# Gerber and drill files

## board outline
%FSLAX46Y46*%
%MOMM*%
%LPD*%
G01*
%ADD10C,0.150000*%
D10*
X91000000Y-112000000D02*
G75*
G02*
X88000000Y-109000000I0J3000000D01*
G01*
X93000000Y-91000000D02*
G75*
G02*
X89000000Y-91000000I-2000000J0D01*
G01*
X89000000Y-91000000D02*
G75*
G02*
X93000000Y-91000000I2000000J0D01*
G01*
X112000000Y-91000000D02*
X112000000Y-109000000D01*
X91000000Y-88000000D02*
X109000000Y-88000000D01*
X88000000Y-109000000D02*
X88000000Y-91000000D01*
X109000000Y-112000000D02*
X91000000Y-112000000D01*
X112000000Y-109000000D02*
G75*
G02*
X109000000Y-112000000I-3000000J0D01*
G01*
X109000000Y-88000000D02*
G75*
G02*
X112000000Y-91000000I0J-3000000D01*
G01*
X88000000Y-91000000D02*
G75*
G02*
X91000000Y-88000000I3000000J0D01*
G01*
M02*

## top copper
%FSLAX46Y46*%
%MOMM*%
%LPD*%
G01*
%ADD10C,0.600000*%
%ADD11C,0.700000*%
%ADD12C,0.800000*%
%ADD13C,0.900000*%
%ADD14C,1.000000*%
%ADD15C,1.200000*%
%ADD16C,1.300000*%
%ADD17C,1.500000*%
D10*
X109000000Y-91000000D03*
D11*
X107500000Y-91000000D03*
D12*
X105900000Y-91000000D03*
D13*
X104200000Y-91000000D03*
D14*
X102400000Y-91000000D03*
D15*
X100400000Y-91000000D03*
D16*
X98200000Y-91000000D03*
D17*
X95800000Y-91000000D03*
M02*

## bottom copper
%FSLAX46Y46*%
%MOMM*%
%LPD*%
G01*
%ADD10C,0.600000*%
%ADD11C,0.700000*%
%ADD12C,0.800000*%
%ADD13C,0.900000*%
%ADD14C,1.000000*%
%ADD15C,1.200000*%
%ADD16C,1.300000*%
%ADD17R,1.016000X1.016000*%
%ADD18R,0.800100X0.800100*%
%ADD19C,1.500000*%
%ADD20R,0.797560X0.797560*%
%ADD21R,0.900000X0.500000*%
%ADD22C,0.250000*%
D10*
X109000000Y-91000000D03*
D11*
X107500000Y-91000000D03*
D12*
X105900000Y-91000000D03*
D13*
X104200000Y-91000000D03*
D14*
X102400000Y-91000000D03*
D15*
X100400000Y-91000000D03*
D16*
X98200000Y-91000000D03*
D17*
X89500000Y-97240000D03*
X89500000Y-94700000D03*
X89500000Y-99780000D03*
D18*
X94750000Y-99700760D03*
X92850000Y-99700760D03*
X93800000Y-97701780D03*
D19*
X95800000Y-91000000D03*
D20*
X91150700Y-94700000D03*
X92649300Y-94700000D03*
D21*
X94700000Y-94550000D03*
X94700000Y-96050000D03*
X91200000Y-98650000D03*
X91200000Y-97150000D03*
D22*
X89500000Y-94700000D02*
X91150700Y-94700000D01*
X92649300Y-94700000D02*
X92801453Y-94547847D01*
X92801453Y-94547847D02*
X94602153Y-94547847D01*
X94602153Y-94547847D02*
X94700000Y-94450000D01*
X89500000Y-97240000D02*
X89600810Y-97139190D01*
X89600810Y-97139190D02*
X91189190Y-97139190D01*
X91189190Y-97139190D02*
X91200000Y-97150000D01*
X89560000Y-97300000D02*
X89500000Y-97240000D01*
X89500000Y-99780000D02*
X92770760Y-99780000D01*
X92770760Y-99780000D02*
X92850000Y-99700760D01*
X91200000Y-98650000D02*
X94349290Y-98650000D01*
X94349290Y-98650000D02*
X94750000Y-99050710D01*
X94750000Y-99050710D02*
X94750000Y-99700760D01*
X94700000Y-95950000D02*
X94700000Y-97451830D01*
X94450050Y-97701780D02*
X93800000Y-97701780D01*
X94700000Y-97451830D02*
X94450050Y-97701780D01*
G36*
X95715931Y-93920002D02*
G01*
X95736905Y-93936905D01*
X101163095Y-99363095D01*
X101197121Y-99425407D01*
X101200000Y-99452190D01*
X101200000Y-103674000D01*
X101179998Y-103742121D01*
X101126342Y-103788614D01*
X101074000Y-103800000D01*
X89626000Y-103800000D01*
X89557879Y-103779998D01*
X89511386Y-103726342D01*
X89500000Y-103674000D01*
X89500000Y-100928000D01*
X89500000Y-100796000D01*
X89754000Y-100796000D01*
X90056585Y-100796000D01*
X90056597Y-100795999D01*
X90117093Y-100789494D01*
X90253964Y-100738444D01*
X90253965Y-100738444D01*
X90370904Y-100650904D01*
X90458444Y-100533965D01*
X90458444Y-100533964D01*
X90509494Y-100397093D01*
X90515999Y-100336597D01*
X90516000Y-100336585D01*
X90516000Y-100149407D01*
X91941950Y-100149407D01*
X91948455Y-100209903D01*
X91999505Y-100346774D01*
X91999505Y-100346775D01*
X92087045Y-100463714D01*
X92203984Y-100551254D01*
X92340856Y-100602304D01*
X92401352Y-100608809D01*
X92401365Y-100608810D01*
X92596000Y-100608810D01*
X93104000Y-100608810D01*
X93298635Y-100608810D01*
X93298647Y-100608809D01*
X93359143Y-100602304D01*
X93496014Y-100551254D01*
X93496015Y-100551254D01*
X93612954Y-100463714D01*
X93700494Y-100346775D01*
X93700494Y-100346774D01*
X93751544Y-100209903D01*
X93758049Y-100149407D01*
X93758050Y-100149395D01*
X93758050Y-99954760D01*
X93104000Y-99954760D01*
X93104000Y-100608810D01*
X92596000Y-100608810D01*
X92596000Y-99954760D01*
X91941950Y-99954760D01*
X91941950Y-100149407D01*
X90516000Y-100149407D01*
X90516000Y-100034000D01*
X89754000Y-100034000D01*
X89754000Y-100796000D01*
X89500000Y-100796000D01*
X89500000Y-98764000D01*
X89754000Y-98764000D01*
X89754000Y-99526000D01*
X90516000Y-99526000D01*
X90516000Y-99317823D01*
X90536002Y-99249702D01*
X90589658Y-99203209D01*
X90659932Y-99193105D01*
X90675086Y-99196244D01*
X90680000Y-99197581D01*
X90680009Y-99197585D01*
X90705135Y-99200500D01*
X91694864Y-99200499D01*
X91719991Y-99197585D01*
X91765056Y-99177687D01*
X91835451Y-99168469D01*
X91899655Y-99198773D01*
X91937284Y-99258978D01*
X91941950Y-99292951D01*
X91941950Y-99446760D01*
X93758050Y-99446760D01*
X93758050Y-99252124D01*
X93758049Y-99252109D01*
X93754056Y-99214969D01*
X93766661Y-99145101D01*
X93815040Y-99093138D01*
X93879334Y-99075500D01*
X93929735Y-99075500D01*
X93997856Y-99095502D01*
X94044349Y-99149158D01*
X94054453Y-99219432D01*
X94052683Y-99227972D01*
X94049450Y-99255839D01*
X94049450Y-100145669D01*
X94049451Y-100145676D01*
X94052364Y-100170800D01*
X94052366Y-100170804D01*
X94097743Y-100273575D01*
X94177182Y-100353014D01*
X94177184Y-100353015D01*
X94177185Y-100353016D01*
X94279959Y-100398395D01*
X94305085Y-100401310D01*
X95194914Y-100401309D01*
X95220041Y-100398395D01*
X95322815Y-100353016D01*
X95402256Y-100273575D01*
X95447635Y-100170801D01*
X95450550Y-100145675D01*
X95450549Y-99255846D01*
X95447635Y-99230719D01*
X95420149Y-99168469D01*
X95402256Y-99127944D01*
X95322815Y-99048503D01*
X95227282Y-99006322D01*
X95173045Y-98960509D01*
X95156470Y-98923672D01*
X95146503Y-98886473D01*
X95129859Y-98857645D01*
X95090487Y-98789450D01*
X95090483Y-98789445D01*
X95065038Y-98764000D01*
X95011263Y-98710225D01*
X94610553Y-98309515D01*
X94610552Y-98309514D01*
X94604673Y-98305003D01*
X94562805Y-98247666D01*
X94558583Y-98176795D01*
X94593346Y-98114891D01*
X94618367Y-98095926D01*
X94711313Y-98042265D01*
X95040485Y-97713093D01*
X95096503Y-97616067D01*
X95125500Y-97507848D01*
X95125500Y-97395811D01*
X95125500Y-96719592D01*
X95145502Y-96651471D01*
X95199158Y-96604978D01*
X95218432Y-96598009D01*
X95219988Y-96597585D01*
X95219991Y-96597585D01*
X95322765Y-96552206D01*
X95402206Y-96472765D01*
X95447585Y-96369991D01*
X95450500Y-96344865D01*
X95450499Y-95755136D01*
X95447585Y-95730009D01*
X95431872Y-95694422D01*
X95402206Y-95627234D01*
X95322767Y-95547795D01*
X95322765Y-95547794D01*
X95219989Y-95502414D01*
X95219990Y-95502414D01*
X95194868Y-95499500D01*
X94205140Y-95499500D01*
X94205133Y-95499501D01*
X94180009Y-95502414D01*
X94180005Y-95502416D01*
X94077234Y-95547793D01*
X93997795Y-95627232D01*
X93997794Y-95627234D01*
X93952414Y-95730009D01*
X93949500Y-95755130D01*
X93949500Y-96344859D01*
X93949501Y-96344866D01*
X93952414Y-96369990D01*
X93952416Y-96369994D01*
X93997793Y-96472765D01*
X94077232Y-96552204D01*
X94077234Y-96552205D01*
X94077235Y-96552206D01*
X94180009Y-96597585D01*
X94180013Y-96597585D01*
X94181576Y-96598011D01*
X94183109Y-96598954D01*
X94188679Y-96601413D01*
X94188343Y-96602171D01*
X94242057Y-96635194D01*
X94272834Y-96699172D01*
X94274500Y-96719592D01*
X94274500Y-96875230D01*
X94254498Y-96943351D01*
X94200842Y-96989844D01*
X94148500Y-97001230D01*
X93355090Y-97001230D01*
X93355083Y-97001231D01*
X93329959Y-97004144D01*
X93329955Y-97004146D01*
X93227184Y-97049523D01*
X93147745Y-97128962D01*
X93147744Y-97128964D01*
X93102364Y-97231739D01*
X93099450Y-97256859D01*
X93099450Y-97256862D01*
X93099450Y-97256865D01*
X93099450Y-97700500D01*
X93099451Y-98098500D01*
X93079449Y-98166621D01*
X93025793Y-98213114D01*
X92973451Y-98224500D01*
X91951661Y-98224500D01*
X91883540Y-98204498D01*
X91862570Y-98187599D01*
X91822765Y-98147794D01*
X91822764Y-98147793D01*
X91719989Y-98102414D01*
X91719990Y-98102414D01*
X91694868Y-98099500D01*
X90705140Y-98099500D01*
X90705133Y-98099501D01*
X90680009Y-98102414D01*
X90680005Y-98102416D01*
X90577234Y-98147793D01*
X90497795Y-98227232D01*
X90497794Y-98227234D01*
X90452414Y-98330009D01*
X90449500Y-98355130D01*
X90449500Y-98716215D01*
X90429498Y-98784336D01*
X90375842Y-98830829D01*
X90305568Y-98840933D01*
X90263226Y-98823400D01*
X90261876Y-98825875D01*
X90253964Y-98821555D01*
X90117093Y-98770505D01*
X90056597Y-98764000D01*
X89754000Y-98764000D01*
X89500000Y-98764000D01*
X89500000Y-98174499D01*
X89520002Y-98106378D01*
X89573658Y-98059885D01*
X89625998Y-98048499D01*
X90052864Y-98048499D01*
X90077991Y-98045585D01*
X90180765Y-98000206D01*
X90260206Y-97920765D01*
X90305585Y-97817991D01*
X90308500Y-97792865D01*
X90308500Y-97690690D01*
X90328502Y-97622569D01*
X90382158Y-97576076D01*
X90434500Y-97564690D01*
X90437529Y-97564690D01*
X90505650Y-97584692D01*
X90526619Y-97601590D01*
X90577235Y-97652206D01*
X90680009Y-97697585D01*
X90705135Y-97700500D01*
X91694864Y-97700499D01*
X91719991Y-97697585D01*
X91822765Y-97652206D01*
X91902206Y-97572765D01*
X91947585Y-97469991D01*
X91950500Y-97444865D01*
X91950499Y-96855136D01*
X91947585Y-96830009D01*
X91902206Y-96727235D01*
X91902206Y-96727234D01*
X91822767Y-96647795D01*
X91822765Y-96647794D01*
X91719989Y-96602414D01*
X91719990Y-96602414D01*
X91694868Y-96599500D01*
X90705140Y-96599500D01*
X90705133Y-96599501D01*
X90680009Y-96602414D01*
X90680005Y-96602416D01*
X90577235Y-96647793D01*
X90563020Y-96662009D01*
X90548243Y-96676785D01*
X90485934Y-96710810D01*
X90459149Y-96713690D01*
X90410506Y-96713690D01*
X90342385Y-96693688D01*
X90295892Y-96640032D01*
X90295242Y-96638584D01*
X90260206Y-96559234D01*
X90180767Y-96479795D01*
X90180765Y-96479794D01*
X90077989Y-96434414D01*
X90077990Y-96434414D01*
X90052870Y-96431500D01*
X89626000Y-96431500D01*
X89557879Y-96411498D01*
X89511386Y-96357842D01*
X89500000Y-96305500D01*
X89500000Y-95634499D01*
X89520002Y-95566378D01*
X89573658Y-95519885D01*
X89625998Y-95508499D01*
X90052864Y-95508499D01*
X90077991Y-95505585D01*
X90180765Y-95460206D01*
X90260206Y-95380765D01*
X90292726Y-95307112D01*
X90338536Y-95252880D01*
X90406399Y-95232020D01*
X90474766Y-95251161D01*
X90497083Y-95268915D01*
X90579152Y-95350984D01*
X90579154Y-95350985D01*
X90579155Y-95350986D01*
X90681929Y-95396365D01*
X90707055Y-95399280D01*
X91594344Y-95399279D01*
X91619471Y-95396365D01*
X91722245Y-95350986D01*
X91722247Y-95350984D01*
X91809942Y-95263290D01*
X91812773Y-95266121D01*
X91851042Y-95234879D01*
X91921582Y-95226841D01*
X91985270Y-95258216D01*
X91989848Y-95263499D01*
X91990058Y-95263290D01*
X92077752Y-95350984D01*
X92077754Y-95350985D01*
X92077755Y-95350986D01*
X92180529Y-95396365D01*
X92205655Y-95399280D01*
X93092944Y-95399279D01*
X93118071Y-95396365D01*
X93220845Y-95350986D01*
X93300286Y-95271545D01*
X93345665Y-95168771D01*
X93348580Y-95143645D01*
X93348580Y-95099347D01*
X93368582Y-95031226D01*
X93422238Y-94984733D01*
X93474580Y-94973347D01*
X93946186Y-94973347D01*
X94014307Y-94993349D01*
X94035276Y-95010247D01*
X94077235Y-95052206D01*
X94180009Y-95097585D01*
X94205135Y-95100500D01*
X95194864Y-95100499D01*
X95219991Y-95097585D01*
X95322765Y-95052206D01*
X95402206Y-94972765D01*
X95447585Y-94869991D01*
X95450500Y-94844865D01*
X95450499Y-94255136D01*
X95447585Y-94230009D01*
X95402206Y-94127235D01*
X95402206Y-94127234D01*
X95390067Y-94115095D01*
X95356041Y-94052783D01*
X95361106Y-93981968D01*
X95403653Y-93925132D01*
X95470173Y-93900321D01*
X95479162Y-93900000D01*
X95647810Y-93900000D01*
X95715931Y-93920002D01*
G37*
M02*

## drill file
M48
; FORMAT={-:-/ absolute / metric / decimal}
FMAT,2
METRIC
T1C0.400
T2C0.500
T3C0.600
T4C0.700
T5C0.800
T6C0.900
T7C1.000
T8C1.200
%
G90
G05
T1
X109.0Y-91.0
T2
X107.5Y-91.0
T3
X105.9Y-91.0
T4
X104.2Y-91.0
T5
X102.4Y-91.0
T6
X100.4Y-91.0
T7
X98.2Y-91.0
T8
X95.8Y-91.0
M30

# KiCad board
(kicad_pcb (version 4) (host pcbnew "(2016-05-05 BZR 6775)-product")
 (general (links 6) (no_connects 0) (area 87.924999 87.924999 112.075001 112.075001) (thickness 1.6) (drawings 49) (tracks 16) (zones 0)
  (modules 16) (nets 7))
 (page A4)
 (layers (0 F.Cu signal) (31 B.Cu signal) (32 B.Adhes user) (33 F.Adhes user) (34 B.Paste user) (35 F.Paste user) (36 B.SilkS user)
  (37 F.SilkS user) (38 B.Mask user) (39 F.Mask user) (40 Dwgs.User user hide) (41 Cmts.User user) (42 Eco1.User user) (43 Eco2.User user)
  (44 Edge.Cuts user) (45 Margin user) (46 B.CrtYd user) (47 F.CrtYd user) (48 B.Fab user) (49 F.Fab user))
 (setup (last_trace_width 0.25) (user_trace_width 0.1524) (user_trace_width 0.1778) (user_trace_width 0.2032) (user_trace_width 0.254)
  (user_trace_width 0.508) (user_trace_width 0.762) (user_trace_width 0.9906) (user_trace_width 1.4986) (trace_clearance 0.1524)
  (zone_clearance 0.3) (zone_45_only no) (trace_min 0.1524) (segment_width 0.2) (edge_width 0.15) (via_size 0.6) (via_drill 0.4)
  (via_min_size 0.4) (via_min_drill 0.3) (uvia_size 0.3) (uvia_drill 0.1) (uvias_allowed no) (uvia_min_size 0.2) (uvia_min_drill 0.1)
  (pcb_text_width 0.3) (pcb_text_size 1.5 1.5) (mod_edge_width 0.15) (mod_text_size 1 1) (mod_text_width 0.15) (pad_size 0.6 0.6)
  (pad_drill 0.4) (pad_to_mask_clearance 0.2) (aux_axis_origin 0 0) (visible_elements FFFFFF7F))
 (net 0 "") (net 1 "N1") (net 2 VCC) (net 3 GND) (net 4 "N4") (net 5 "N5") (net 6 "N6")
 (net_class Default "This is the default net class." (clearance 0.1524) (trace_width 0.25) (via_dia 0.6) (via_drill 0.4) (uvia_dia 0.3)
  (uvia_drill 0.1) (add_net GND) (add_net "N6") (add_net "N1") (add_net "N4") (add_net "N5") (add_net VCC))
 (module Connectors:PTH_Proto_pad (layer F.Cu) (at 109 91)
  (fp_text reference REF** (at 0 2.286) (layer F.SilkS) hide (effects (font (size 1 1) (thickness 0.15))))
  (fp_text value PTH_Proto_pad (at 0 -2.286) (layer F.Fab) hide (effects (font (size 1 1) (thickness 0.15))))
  (pad 1 thru_hole circle (at 0 0) (size 0.6 0.6) (drill 0.4) (layers *.Cu *.Mask F.SilkS)))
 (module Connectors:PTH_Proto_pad (layer F.Cu) (at 107.5 91)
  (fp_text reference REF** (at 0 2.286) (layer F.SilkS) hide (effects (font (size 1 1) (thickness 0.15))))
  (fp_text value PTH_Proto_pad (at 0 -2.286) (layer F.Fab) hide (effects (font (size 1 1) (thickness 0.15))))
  (pad 1 thru_hole circle (at 0 0) (size 0.7 0.7) (drill 0.5) (layers *.Cu *.Mask F.SilkS)))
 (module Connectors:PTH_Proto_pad (layer F.Cu) (at 105.9 91)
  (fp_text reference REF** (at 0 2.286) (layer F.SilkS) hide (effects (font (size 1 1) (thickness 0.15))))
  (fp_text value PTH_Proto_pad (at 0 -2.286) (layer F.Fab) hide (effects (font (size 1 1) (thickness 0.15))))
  (pad 1 thru_hole circle (at 0 0) (size 0.8 0.8) (drill 0.6) (layers *.Cu *.Mask F.SilkS)))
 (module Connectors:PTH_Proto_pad (layer F.Cu) (at 104.2 91)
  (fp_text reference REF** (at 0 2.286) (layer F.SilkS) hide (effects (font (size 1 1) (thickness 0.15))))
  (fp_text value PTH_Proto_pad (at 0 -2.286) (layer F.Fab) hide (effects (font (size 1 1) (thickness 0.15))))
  (pad 1 thru_hole circle (at 0 0) (size 0.9 0.9) (drill 0.7) (layers *.Cu *.Mask F.SilkS)))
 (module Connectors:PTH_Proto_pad (layer F.Cu) (at 102.4 91)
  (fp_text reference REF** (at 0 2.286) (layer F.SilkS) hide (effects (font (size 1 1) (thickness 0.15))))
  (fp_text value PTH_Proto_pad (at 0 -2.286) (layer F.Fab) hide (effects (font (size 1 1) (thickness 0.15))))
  (pad 1 thru_hole circle (at 0 0) (size 1 1) (drill 0.8) (layers *.Cu *.Mask F.SilkS)))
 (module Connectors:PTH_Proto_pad (layer F.Cu) (at 100.4 91)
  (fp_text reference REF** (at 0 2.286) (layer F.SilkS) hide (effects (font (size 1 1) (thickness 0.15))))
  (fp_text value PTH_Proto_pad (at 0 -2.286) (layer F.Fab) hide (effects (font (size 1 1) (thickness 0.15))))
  (pad 1 thru_hole circle (at 0 0) (size 1.2 1.2) (drill 0.9) (layers *.Cu *.Mask F.SilkS)))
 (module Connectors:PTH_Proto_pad (layer F.Cu) (at 98.2 91)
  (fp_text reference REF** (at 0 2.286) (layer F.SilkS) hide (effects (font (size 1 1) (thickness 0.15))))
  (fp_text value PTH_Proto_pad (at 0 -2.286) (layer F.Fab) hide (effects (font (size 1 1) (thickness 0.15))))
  (pad 1 thru_hole circle (at 0 0) (size 1.3 1.3) (drill 1) (layers *.Cu *.Mask F.SilkS)))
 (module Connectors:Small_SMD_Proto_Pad (layer B.Cu) (at 89.5 97.24)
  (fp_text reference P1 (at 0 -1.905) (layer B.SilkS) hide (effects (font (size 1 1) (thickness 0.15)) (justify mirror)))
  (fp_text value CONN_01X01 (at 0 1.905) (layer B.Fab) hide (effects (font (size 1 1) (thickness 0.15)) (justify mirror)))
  (pad 1 smd rect (at 0 0) (size 1.016 1.016) (layers B.Cu B.Paste B.Mask) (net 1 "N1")))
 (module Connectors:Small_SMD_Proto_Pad (layer B.Cu) (at 89.5 94.7)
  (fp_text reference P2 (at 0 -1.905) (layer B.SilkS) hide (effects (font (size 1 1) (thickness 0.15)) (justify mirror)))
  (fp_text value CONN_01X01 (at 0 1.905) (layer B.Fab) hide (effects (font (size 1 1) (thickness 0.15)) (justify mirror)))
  (pad 1 smd rect (at 0 0) (size 1.016 1.016) (layers B.Cu B.Paste B.Mask) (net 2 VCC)))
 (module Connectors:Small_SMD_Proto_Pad (layer B.Cu) (at 89.5 99.78)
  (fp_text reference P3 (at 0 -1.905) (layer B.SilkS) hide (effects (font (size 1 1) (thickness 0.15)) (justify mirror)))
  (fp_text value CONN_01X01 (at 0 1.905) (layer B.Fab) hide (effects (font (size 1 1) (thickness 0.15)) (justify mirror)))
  (pad 1 smd rect (at 0 0) (size 1.016 1.016) (layers B.Cu B.Paste B.Mask) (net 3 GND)))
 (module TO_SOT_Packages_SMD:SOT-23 (layer B.Cu) (at 93.8 98.7 180)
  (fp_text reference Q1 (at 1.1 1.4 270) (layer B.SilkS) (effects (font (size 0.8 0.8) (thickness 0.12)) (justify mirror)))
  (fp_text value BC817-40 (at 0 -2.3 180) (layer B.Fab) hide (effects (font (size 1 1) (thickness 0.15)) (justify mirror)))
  (pad 1 smd rect (at -0.95 -1.00076 180) (size 0.8001 0.8001) (layers B.Cu B.Paste B.Mask) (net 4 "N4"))
  (pad 2 smd rect (at 0.95 -1.00076 180) (size 0.8001 0.8001) (layers B.Cu B.Paste B.Mask) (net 3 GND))
  (pad 3 smd rect (at 0 0.99822 180) (size 0.8001 0.8001) (layers B.Cu B.Paste B.Mask) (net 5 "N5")))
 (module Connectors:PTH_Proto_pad (layer F.Cu) (at 95.8 91)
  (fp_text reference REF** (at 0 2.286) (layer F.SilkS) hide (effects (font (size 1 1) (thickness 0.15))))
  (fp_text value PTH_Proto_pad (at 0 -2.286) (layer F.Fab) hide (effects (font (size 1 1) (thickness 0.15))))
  (pad 1 thru_hole circle (at 0 0) (size 1.5 1.5) (drill 1.2) (layers *.Cu *.Mask F.SilkS)))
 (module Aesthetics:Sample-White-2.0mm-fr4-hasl (layer B.Cu) (at 100 102.6 180)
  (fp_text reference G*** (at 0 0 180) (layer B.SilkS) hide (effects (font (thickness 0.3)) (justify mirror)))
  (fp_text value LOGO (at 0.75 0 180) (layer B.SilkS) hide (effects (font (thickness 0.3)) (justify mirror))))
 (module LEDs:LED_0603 (layer B.Cu) (at 91.9 94.7 180)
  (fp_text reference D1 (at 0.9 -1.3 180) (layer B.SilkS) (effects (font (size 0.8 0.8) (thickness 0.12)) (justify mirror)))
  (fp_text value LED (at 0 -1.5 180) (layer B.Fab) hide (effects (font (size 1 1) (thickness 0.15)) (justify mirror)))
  (pad 2 smd rect (at 0.7493 0) (size 0.79756 0.79756) (layers B.Cu B.Paste B.Mask) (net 2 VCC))
  (pad 1 smd rect (at -0.7493 0) (size 0.79756 0.79756) (layers B.Cu B.Paste B.Mask) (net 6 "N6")))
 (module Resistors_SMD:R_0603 (layer B.Cu) (at 94.7 95.3 270)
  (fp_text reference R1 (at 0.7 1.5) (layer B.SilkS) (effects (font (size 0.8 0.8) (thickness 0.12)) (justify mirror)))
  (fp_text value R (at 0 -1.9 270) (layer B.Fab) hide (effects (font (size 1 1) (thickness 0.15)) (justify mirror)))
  (pad 1 smd rect (at -0.75 0 270) (size 0.5 0.9) (layers B.Cu B.Paste B.Mask) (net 6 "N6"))
  (pad 2 smd rect (at 0.75 0 270) (size 0.5 0.9) (layers B.Cu B.Paste B.Mask) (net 5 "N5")))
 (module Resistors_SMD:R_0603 (layer B.Cu) (at 91.2 97.9 90)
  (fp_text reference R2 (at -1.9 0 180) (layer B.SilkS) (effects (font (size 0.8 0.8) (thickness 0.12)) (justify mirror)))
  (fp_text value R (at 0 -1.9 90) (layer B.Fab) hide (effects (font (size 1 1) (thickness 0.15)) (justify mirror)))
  (pad 1 smd rect (at -0.75 0 90) (size 0.5 0.9) (layers B.Cu B.Paste B.Mask) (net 4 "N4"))
  (pad 2 smd rect (at 0.75 0 90) (size 0.5 0.9) (layers B.Cu B.Paste B.Mask) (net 1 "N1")))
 (gr_arc (start 91 109) (end 91 112) (angle 90) (layer Edge.Cuts) (width 0.15))
 (gr_circle (center 91 91) (end 93 91) (layer Edge.Cuts) (width 0.15))
 (gr_line (start 112 91) (end 112 109) (layer Edge.Cuts) (width 0.15))
 (gr_line (start 91 88) (end 109 88) (layer Edge.Cuts) (width 0.15))
 (gr_line (start 88 109) (end 88 91) (layer Edge.Cuts) (width 0.15))
 (gr_line (start 109 112) (end 91 112) (layer Edge.Cuts) (width 0.15))
 (gr_arc (start 109 109) (end 112 109) (angle 90) (layer Edge.Cuts) (width 0.15))
 (gr_arc (start 109 91) (end 109 88) (angle 90) (layer Edge.Cuts) (width 0.15))
 (gr_arc (start 91 91) (end 88 91) (angle 90) (layer Edge.Cuts) (width 0.15))
 (segment (start 89.5 94.7) (end 91.1507 94.7) (width 0.25) (layer B.Cu) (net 2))
 (segment (start 92.6493 94.7) (end 92.801453 94.547847) (width 0.25) (layer B.Cu) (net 6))
 (segment (start 92.801453 94.547847) (end 94.602153 94.547847) (width 0.25) (layer B.Cu) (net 6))
 (segment (start 94.602153 94.547847) (end 94.7 94.45) (width 0.25) (layer B.Cu) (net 6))
 (segment (start 89.5 97.24) (end 89.60081 97.13919) (width 0.25) (layer B.Cu) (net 1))
 (segment (start 89.60081 97.13919) (end 91.18919 97.13919) (width 0.25) (layer B.Cu) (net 1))
 (segment (start 91.18919 97.13919) (end 91.2 97.15) (width 0.25) (layer B.Cu) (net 1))
 (segment (start 89.56 97.3) (end 89.5 97.24) (width 0.25) (layer B.Cu) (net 1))
 (segment (start 89.5 99.78) (end 92.77076 99.78) (width 0.25) (layer B.Cu) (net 3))
 (segment (start 92.77076 99.78) (end 92.85 99.70076) (width 0.25) (layer B.Cu) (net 3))
 (segment (start 91.2 98.65) (end 94.34929 98.65) (width 0.25) (layer B.Cu) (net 4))
 (segment (start 94.34929 98.65) (end 94.75 99.05071) (width 0.25) (layer B.Cu) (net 4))
 (segment (start 94.75 99.05071) (end 94.75 99.70076) (width 0.25) (layer B.Cu) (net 4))
 (segment (start 94.7 95.95) (end 94.7 97.45183) (width 0.25) (layer B.Cu) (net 5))
 (segment (start 94.45005 97.70178) (end 93.8 97.70178) (width 0.25) (layer B.Cu) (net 5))
 (segment (start 94.7 97.45183) (end 94.45005 97.70178) (width 0.25) (layer B.Cu) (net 5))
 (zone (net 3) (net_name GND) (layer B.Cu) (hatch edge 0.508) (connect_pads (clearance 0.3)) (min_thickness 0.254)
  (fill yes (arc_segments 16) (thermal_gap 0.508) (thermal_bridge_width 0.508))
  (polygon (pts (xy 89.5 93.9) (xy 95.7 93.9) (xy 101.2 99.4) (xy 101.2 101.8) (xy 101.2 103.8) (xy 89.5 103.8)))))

